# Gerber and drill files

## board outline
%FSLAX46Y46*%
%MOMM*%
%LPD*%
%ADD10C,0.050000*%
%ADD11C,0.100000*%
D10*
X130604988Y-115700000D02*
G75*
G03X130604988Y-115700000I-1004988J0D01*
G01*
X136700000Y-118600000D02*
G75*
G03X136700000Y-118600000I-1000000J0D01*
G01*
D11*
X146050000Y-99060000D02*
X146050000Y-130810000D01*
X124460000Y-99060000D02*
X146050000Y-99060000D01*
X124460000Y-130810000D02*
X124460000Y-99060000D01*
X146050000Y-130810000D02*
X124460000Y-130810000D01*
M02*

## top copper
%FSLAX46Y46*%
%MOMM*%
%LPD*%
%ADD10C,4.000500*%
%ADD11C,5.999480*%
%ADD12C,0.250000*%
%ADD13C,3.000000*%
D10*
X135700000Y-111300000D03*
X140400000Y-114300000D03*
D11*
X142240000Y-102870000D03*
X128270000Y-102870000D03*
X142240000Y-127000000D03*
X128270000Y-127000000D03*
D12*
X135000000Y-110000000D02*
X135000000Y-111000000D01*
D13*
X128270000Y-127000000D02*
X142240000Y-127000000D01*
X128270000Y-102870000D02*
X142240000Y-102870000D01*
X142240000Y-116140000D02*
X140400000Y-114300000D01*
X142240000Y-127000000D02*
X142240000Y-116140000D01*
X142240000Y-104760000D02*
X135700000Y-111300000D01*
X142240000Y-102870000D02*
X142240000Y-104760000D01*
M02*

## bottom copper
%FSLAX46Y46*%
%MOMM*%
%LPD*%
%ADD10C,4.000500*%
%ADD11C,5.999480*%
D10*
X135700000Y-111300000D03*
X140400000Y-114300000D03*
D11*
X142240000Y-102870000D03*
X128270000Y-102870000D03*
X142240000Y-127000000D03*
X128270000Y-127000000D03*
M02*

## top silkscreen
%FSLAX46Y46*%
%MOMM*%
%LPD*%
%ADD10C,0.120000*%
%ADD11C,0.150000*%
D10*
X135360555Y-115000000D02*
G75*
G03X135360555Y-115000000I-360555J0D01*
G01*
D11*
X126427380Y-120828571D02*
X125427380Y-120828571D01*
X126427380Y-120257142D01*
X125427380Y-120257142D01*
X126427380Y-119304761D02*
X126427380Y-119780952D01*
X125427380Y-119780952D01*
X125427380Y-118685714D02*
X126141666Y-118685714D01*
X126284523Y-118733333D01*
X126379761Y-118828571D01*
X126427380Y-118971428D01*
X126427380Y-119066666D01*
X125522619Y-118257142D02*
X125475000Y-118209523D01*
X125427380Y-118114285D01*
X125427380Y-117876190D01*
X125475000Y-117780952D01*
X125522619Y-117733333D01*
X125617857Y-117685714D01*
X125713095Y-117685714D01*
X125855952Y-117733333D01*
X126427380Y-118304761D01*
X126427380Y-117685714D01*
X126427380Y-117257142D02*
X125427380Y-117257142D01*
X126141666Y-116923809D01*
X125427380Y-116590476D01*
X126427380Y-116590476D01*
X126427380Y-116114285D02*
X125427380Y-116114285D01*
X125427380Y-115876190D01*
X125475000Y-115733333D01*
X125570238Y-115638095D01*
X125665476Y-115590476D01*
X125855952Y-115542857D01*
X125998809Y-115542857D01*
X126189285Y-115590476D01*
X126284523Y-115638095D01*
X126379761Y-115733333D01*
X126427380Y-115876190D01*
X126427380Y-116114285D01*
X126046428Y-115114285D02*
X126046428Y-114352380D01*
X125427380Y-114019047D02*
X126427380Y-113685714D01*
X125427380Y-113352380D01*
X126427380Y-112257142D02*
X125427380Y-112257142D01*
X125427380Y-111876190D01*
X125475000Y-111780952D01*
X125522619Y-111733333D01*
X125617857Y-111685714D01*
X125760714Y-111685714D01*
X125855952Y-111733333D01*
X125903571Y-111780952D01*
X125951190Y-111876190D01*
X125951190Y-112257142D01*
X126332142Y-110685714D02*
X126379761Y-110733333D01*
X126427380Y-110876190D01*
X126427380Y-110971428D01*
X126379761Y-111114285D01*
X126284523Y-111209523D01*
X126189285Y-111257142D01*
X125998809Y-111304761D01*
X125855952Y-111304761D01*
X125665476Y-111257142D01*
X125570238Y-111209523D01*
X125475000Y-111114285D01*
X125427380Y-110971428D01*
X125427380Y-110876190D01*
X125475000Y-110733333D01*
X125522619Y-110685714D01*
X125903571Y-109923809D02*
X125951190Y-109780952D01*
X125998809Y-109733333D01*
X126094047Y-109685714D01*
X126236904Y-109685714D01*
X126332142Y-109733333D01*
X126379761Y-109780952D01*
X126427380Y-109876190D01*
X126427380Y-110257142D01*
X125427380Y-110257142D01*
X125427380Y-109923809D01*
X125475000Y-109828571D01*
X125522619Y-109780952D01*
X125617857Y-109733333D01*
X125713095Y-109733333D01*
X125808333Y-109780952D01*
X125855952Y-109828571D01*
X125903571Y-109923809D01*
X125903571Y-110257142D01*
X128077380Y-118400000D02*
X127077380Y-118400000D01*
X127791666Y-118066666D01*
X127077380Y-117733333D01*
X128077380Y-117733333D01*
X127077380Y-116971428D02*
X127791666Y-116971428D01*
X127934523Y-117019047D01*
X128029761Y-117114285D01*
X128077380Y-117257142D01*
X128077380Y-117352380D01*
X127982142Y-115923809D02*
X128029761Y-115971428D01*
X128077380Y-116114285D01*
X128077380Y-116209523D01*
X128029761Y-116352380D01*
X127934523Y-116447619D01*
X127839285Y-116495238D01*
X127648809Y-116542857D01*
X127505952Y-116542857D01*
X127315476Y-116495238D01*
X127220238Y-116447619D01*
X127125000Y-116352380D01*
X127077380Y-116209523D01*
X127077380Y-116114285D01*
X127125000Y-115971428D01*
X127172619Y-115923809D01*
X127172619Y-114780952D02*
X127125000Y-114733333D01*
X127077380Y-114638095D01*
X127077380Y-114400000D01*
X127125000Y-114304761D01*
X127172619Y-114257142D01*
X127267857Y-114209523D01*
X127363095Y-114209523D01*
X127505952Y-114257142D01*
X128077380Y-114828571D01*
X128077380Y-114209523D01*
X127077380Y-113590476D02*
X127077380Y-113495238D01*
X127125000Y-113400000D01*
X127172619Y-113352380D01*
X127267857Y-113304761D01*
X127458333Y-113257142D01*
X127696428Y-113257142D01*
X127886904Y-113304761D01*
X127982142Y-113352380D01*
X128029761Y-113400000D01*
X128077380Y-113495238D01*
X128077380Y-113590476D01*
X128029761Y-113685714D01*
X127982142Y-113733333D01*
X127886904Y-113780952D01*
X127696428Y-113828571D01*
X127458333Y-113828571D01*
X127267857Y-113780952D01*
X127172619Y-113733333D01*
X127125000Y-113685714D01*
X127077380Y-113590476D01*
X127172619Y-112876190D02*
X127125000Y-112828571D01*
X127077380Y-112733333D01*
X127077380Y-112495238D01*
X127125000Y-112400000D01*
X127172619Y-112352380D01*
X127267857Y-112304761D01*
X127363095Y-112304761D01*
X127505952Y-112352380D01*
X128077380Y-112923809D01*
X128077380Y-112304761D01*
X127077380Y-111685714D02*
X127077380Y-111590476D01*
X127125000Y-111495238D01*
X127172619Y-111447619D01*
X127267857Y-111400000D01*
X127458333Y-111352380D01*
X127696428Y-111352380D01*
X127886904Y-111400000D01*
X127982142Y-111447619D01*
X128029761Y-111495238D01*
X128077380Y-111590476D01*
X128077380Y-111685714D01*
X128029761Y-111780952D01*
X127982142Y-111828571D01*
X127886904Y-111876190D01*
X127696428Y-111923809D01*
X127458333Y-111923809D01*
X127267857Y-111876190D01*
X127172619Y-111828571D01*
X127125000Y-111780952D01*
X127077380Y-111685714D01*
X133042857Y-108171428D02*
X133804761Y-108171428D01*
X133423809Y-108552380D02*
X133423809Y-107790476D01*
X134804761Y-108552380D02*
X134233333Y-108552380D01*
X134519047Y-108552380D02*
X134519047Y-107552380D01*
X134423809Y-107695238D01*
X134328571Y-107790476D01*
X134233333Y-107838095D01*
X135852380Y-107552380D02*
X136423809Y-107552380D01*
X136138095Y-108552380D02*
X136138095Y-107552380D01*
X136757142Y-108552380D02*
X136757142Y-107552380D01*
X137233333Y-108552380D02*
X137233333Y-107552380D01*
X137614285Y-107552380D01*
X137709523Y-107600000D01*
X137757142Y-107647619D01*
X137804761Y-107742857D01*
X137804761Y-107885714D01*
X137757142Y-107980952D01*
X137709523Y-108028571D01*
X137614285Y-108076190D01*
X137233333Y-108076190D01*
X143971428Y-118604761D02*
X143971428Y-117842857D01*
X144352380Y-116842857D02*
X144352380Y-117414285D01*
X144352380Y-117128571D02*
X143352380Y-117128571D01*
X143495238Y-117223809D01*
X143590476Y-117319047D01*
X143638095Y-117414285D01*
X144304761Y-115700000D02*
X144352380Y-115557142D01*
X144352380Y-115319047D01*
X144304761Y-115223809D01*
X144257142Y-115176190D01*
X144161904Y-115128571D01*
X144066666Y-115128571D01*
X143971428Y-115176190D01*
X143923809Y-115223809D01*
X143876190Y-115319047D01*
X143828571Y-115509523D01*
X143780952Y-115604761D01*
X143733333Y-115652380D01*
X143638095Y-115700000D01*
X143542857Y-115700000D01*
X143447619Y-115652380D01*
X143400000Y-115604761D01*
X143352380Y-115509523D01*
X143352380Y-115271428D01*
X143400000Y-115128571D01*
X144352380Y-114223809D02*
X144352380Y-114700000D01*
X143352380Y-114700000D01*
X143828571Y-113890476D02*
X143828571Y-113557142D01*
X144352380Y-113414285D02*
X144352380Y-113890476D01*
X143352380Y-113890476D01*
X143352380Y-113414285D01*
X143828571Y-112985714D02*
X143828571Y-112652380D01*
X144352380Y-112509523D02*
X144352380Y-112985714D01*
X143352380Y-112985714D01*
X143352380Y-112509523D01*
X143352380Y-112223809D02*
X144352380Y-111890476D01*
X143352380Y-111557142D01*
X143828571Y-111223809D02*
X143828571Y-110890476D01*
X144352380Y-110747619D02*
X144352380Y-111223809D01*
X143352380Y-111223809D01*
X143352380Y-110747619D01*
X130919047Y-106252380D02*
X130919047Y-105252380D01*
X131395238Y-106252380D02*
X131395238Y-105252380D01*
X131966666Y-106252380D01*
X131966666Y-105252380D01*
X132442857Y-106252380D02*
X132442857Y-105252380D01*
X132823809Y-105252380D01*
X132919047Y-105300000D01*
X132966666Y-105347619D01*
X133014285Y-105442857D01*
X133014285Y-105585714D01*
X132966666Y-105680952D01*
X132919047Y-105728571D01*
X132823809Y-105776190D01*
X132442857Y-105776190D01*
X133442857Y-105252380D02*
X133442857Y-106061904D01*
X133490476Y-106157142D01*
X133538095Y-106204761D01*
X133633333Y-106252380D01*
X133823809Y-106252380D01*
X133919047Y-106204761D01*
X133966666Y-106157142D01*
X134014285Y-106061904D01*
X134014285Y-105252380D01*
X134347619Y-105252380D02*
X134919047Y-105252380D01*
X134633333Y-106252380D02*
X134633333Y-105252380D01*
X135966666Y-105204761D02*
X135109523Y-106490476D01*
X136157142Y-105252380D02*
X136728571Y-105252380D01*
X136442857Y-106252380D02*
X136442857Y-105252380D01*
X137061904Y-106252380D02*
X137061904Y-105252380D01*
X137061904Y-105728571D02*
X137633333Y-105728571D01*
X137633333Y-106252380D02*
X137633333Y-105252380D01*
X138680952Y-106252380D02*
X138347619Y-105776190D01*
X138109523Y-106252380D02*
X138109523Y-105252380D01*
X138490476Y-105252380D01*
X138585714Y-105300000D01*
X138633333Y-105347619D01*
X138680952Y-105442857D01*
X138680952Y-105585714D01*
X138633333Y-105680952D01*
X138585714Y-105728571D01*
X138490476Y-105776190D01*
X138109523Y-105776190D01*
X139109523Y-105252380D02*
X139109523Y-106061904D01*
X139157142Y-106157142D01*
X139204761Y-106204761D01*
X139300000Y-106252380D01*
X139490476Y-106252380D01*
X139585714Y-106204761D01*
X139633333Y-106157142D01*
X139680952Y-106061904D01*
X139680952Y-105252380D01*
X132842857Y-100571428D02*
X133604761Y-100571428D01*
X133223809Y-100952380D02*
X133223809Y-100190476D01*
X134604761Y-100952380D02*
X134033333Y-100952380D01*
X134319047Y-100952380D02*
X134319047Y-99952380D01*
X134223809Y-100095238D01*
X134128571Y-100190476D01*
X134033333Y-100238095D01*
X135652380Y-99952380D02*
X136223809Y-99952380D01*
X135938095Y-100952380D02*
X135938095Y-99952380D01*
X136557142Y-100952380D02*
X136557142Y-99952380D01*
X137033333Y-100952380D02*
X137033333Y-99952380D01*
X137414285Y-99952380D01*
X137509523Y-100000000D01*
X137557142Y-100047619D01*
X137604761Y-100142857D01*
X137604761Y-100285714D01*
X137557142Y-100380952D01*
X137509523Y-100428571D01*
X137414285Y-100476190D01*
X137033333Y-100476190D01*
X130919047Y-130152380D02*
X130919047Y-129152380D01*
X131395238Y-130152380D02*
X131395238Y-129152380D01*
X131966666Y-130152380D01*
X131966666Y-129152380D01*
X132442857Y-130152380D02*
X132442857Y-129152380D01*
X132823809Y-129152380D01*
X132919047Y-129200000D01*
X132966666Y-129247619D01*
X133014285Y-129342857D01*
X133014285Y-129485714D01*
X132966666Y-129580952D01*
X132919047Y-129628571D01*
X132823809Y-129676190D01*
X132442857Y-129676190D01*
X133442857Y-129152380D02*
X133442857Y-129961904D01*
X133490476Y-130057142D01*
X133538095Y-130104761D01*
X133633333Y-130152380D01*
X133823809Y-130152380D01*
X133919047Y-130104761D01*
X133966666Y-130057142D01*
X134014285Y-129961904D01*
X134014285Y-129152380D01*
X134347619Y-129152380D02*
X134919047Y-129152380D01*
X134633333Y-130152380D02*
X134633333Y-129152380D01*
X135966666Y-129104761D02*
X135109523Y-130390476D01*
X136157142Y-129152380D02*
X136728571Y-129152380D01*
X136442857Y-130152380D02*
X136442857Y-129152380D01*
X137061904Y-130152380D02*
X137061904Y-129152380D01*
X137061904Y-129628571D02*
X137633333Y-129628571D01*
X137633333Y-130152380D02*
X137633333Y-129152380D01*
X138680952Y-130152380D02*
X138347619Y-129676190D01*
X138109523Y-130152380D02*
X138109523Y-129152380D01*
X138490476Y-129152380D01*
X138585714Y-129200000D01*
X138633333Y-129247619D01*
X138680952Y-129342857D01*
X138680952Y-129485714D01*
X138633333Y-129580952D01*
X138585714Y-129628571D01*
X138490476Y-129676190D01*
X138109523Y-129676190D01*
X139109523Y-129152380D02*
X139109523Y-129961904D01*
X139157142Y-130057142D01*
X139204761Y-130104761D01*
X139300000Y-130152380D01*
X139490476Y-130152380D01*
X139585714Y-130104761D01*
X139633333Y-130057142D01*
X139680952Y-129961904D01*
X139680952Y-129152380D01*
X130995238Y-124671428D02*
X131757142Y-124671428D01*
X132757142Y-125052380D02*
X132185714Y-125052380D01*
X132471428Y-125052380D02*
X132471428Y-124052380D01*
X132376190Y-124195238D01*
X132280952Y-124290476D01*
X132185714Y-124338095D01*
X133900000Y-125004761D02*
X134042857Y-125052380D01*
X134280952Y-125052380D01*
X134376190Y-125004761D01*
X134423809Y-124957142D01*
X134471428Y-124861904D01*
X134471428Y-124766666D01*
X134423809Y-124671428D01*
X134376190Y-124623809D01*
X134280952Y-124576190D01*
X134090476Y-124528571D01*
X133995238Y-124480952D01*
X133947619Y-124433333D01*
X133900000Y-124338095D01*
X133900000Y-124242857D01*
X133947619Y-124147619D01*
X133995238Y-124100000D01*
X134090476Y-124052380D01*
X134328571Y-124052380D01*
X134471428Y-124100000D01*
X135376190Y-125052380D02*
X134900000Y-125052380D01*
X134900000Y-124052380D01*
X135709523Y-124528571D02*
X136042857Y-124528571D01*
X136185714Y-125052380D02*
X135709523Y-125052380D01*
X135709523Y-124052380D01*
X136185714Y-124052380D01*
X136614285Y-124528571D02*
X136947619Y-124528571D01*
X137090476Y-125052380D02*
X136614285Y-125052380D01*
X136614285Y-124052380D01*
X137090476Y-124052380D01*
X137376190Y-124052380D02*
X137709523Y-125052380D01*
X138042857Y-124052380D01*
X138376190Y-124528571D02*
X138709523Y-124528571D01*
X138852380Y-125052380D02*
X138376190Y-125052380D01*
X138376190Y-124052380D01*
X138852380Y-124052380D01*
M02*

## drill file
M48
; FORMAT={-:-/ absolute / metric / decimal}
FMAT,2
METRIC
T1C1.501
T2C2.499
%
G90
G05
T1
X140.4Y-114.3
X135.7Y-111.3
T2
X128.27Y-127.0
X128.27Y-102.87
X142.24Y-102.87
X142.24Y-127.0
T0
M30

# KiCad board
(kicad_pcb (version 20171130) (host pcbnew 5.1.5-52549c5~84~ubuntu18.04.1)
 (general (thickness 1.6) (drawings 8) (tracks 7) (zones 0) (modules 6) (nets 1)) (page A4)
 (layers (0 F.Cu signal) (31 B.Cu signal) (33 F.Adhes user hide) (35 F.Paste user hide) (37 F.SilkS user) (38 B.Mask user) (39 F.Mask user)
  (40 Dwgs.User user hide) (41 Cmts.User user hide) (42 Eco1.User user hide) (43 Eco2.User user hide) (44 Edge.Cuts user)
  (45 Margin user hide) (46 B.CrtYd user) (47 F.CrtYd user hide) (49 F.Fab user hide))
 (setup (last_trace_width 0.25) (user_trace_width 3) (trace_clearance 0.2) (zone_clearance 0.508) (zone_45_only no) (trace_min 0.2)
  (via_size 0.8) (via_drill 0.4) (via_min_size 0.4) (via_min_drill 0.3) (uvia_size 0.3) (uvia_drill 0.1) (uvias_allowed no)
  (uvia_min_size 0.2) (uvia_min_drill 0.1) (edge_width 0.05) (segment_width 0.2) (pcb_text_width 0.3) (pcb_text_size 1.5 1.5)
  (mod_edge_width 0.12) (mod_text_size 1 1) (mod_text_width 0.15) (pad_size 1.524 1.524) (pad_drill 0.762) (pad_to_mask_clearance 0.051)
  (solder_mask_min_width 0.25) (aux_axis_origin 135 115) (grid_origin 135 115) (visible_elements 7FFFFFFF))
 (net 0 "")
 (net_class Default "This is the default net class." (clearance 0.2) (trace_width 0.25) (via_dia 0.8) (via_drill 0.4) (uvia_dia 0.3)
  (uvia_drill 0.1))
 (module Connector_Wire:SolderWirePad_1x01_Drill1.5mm (layer F.Cu) (at 135.7 111.3)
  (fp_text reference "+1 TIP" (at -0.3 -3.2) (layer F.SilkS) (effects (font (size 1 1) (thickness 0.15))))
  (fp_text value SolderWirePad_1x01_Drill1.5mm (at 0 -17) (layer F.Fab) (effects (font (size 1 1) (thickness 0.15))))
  (pad 1 thru_hole circle (at 0 0) (size 4.0005 4.0005) (drill 1.50114) (layers *.Cu *.Mask)))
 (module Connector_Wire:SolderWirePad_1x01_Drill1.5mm (layer F.Cu) (at 140.4 114.3)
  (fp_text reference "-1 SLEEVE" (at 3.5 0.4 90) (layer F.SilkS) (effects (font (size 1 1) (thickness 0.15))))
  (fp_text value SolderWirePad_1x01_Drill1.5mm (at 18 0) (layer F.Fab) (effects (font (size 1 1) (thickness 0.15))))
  (pad 1 thru_hole circle (at 0 0) (size 4.0005 4.0005) (drill 1.50114) (layers *.Cu *.Mask)))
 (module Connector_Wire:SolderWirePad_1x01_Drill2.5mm (layer F.Cu) (at 142.24 102.87)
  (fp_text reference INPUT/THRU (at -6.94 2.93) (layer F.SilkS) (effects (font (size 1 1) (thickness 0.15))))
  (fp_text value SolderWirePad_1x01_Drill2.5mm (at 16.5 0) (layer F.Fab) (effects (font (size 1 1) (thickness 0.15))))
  (pad 1 thru_hole circle (at 0 0) (size 5.99948 5.99948) (drill 2.49936) (layers *.Cu *.Mask)))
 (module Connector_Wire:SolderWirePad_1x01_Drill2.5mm (layer F.Cu) (at 128.27 102.87)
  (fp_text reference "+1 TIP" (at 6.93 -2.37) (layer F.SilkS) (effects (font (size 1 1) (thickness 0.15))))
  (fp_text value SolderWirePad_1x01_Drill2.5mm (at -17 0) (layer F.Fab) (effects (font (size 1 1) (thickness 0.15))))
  (pad 1 thru_hole circle (at 0 0) (size 5.99948 5.99948) (drill 2.49936) (layers *.Cu *.Mask)))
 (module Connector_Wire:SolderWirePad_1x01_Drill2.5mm (layer F.Cu) (at 142.24 127)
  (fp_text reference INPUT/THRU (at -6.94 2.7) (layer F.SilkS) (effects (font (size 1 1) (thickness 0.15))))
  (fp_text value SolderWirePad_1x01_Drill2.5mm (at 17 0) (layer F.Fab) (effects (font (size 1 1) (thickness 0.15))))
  (pad 1 thru_hole circle (at 0 0) (size 5.99948 5.99948) (drill 2.49936) (layers *.Cu *.Mask)))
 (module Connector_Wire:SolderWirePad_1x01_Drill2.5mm (layer F.Cu) (at 128.27 127)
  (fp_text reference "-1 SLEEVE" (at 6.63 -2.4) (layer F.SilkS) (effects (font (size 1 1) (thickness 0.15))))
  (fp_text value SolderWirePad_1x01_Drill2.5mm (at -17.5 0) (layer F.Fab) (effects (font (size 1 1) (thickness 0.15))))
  (pad 1 thru_hole circle (at 0 0) (size 5.99948 5.99948) (drill 2.49936) (layers *.Cu *.Mask)))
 (gr_circle (center 129.6 115.7) (end 130.6 115.8) (layer Edge.Cuts) (width 0.05))
 (gr_circle (center 135.7 118.6) (end 136.7 118.6) (layer Edge.Cuts) (width 0.05))
 (gr_circle (center 135 115) (end 135.3 115.2) (layer F.SilkS) (width 0.12))
 (gr_line (start 146.05 99.06) (end 146.05 130.81) (layer Edge.Cuts) (width 0.1))
 (gr_line (start 124.46 99.06) (end 146.05 99.06) (layer Edge.Cuts) (width 0.1))
 (gr_line (start 124.46 130.81) (end 124.46 99.06) (layer Edge.Cuts) (width 0.1))
 (gr_line (start 146.05 130.81) (end 124.46 130.81) (layer Edge.Cuts) (width 0.1))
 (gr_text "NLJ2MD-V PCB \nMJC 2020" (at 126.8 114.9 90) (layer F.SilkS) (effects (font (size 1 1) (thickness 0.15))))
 (segment (start 135 110) (end 135 111) (width 0.25) (layer F.Cu) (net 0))
 (segment (start 128.27 127) (end 142.24 127) (width 3) (layer F.Cu) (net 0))
 (segment (start 128.27 102.87) (end 142.24 102.87) (width 3) (layer F.Cu) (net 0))
 (segment (start 142.24 116.14) (end 140.4 114.3) (width 3) (layer F.Cu) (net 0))
 (segment (start 142.24 127) (end 142.24 116.14) (width 3) (layer F.Cu) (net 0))
 (segment (start 142.24 104.76) (end 135.7 111.3) (width 3) (layer F.Cu) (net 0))
 (segment (start 142.24 102.87) (end 142.24 104.76) (width 3) (layer F.Cu) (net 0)))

